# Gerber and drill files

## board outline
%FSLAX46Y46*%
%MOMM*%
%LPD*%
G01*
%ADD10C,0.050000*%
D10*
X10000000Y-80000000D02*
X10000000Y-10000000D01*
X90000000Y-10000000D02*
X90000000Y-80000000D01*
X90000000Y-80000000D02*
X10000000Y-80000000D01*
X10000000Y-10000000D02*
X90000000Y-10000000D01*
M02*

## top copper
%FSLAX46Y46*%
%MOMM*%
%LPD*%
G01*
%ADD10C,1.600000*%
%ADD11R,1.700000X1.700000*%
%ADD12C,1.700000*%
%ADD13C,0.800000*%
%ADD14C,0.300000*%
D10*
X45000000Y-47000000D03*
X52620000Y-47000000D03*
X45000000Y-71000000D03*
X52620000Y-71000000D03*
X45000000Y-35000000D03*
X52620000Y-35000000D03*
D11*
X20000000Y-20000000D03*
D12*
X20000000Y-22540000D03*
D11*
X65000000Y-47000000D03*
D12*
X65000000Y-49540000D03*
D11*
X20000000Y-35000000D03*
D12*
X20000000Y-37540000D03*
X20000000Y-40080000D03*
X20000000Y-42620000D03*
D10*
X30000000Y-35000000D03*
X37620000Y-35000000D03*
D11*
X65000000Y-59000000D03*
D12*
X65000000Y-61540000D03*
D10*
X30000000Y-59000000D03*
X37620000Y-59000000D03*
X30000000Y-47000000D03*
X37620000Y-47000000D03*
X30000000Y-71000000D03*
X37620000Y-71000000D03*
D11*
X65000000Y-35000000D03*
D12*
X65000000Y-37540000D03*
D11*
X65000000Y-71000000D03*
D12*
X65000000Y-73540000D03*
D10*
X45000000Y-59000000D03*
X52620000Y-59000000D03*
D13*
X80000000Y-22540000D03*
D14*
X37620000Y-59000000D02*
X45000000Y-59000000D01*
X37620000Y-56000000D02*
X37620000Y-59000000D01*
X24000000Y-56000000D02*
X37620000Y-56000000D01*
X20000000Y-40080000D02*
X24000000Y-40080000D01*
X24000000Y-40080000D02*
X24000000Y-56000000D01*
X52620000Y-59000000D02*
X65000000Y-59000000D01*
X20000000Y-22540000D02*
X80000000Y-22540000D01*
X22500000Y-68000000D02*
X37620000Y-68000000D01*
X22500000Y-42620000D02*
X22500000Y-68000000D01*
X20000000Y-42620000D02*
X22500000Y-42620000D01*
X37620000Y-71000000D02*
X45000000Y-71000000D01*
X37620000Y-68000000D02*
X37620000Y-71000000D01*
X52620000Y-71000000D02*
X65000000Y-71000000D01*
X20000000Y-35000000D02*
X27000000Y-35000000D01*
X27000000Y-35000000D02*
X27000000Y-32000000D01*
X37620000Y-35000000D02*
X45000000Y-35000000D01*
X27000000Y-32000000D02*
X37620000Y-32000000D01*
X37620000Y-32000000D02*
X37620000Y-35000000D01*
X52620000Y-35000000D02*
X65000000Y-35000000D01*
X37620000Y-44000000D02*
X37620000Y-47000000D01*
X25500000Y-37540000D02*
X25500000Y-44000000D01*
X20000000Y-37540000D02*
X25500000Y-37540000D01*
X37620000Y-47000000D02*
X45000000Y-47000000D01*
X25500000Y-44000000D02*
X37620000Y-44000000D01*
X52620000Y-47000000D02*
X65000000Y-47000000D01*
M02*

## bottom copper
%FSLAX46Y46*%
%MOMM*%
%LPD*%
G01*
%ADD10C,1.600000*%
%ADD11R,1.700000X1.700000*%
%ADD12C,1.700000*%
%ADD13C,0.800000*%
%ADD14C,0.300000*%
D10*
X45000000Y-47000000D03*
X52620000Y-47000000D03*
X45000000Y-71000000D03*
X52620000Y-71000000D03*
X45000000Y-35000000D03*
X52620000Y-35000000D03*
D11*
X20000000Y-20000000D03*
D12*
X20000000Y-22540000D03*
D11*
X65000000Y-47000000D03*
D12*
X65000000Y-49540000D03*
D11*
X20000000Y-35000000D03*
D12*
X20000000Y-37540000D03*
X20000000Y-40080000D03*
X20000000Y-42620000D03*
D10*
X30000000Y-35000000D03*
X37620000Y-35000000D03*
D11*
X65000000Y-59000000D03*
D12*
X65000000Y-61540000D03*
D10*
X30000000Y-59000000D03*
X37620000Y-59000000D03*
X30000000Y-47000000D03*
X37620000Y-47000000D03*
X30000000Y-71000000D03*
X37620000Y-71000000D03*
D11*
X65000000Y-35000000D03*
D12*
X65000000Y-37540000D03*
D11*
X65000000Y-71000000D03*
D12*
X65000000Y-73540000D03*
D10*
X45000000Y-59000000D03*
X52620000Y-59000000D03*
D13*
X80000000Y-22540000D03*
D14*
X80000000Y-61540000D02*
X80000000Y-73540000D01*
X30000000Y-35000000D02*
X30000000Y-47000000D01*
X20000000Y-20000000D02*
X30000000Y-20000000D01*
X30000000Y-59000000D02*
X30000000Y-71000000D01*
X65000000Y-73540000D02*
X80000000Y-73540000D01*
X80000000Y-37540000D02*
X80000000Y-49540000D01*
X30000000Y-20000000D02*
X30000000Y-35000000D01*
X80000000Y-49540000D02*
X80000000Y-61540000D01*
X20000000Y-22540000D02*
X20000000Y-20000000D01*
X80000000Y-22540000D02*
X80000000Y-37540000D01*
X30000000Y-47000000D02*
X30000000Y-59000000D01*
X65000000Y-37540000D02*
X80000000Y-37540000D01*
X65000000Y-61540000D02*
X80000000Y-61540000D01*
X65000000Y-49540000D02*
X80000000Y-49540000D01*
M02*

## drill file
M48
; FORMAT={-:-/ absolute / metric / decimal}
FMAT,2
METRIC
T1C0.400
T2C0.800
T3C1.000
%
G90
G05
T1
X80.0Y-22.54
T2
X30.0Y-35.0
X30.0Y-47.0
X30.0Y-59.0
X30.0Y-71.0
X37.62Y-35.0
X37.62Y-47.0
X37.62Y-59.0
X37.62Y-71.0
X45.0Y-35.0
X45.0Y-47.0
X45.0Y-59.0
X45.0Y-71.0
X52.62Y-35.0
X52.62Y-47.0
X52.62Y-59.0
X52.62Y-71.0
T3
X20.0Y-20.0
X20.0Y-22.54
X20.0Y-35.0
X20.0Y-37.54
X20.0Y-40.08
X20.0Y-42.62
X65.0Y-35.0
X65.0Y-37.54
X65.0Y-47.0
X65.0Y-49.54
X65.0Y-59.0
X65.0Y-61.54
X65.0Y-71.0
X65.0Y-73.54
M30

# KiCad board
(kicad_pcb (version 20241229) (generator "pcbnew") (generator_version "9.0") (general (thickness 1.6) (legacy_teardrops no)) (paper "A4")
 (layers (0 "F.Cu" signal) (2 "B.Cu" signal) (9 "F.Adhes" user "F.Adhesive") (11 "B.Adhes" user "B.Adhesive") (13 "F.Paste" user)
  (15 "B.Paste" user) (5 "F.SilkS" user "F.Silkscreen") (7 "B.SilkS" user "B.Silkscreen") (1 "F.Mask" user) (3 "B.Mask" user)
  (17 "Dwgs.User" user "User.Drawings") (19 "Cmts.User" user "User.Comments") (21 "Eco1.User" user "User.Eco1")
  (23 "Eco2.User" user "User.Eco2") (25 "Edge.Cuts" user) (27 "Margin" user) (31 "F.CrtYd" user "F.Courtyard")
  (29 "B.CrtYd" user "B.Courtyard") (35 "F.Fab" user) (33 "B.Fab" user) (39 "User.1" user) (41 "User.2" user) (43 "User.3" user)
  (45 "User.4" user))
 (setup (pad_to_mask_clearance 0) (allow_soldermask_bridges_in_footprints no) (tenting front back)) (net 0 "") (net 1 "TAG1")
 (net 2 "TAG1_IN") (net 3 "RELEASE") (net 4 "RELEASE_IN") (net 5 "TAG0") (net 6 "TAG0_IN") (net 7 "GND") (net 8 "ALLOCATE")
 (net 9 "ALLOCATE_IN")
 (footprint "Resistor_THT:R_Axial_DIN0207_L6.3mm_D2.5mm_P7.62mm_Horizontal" (layer "F.Cu") (at 45 47)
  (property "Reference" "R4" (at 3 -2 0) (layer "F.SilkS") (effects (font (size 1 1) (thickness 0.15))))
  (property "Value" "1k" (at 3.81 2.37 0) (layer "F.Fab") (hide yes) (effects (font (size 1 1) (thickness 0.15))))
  (pad "1" thru_hole circle (at 0 0) (size 1.6 1.6) (drill 0.8) (layers "*.Cu" "*.Mask") (remove_unused_layers no) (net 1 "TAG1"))
  (pad "2" thru_hole circle (at 7.62 0) (size 1.6 1.6) (drill 0.8) (layers "*.Cu" "*.Mask") (remove_unused_layers no) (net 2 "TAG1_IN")))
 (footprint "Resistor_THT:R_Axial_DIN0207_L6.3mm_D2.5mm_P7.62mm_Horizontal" (layer "F.Cu") (at 45 71)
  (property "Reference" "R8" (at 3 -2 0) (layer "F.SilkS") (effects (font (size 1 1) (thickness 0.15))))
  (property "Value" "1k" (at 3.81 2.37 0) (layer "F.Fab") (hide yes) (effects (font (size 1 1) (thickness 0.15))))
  (pad "1" thru_hole circle (at 0 0) (size 1.6 1.6) (drill 0.8) (layers "*.Cu" "*.Mask") (remove_unused_layers no) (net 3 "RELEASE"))
  (pad "2" thru_hole circle (at 7.62 0) (size 1.6 1.6) (drill 0.8) (layers "*.Cu" "*.Mask") (remove_unused_layers no) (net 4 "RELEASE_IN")))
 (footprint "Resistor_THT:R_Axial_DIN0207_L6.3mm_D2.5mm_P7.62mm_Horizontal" (layer "F.Cu") (at 45 35)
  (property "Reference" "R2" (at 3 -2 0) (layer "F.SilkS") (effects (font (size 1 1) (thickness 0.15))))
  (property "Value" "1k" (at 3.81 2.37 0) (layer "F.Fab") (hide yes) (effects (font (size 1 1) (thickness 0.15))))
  (pad "1" thru_hole circle (at 0 0) (size 1.6 1.6) (drill 0.8) (layers "*.Cu" "*.Mask") (remove_unused_layers no) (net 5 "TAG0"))
  (pad "2" thru_hole circle (at 7.62 0) (size 1.6 1.6) (drill 0.8) (layers "*.Cu" "*.Mask") (remove_unused_layers no) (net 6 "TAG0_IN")))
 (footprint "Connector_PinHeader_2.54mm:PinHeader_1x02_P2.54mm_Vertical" (layer "F.Cu") (at 20 20)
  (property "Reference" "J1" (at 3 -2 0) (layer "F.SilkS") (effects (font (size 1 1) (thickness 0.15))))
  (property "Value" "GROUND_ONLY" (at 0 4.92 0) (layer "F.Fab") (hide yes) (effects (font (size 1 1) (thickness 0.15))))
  (pad "1" thru_hole rect (at 0 0) (size 1.7 1.7) (drill 1) (layers "*.Cu" "*.Mask") (remove_unused_layers no) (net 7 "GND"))
  (pad "2" thru_hole circle (at 0 2.54) (size 1.7 1.7) (drill 1) (layers "*.Cu" "*.Mask") (remove_unused_layers no) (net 7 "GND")))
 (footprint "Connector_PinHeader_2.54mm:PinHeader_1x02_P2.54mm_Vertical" (layer "F.Cu") (at 65 47)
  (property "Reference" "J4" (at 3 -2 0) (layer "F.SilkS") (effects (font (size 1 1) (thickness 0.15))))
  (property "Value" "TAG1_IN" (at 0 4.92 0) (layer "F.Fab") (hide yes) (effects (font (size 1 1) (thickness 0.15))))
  (pad "1" thru_hole rect (at 0 0) (size 1.7 1.7) (drill 1) (layers "*.Cu" "*.Mask") (remove_unused_layers no) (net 2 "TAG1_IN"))
  (pad "2" thru_hole circle (at 0 2.54) (size 1.7 1.7) (drill 1) (layers "*.Cu" "*.Mask") (remove_unused_layers no) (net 7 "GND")))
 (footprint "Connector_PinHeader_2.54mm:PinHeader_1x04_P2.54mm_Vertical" (layer "F.Cu") (at 20 35)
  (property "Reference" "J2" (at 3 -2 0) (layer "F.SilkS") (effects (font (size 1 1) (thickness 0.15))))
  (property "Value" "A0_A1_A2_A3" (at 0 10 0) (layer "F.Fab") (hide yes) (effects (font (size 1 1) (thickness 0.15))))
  (pad "1" thru_hole rect (at 0 0) (size 1.7 1.7) (drill 1) (layers "*.Cu" "*.Mask") (remove_unused_layers no) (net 5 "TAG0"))
  (pad "2" thru_hole circle (at 0 2.54) (size 1.7 1.7) (drill 1) (layers "*.Cu" "*.Mask") (remove_unused_layers no) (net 1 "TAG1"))
  (pad "3" thru_hole circle (at 0 5.08) (size 1.7 1.7) (drill 1) (layers "*.Cu" "*.Mask") (remove_unused_layers no) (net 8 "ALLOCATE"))
  (pad "4" thru_hole circle (at 0 7.62) (size 1.7 1.7) (drill 1) (layers "*.Cu" "*.Mask") (remove_unused_layers no) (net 3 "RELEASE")))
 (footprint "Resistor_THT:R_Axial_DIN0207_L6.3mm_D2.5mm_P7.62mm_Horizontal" (layer "F.Cu") (at 30 35)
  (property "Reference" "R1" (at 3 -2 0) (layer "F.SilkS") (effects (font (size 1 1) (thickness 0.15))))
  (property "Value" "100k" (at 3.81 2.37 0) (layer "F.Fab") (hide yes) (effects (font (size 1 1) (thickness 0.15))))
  (pad "1" thru_hole circle (at 0 0) (size 1.6 1.6) (drill 0.8) (layers "*.Cu" "*.Mask") (remove_unused_layers no) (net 7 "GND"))
  (pad "2" thru_hole circle (at 7.62 0) (size 1.6 1.6) (drill 0.8) (layers "*.Cu" "*.Mask") (remove_unused_layers no) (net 5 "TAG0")))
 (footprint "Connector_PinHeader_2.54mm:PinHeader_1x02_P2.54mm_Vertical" (layer "F.Cu") (at 65 59)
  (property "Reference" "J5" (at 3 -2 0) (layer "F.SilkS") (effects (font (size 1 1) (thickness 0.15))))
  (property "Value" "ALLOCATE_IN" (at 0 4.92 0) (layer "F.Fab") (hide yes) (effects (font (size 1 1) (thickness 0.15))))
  (pad "1" thru_hole rect (at 0 0) (size 1.7 1.7) (drill 1) (layers "*.Cu" "*.Mask") (remove_unused_layers no) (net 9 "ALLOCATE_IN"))
  (pad "2" thru_hole circle (at 0 2.54) (size 1.7 1.7) (drill 1) (layers "*.Cu" "*.Mask") (remove_unused_layers no) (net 7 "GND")))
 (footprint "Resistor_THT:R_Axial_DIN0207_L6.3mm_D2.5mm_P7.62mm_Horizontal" (layer "F.Cu") (at 30 59)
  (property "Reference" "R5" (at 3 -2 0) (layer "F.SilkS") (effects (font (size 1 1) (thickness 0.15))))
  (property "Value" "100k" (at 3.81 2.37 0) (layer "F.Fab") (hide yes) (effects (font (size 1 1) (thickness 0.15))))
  (pad "1" thru_hole circle (at 0 0) (size 1.6 1.6) (drill 0.8) (layers "*.Cu" "*.Mask") (remove_unused_layers no) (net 7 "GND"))
  (pad "2" thru_hole circle (at 7.62 0) (size 1.6 1.6) (drill 0.8) (layers "*.Cu" "*.Mask") (remove_unused_layers no) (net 8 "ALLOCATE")))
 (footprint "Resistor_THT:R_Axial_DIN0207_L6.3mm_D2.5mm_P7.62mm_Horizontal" (layer "F.Cu") (at 30 47)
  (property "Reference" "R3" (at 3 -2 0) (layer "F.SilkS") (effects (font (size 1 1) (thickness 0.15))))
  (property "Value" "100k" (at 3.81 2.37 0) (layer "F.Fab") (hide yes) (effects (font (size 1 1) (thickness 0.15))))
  (pad "1" thru_hole circle (at 0 0) (size 1.6 1.6) (drill 0.8) (layers "*.Cu" "*.Mask") (remove_unused_layers no) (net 7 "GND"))
  (pad "2" thru_hole circle (at 7.62 0) (size 1.6 1.6) (drill 0.8) (layers "*.Cu" "*.Mask") (remove_unused_layers no) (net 1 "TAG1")))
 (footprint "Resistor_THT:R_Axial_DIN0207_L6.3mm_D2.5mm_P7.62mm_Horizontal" (layer "F.Cu") (at 30 71)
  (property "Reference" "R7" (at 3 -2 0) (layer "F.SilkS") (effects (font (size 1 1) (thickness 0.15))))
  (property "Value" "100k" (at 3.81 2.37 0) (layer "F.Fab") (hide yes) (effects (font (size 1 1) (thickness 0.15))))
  (pad "1" thru_hole circle (at 0 0) (size 1.6 1.6) (drill 0.8) (layers "*.Cu" "*.Mask") (remove_unused_layers no) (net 7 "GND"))
  (pad "2" thru_hole circle (at 7.62 0) (size 1.6 1.6) (drill 0.8) (layers "*.Cu" "*.Mask") (remove_unused_layers no) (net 3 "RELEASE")))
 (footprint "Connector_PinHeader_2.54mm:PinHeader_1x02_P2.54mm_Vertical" (layer "F.Cu") (at 65 35)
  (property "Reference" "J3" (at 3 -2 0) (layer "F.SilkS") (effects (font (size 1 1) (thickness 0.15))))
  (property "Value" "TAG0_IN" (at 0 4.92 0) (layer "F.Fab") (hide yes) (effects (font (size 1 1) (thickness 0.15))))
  (pad "1" thru_hole rect (at 0 0) (size 1.7 1.7) (drill 1) (layers "*.Cu" "*.Mask") (remove_unused_layers no) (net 6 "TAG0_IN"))
  (pad "2" thru_hole circle (at 0 2.54) (size 1.7 1.7) (drill 1) (layers "*.Cu" "*.Mask") (remove_unused_layers no) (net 7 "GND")))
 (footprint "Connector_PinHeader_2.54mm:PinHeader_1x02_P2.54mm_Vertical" (layer "F.Cu") (at 65 71)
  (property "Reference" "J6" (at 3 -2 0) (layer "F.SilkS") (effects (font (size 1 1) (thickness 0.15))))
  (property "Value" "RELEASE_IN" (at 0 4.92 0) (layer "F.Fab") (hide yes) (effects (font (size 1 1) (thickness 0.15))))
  (pad "1" thru_hole rect (at 0 0) (size 1.7 1.7) (drill 1) (layers "*.Cu" "*.Mask") (remove_unused_layers no) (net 4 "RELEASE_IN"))
  (pad "2" thru_hole circle (at 0 2.54) (size 1.7 1.7) (drill 1) (layers "*.Cu" "*.Mask") (remove_unused_layers no) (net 7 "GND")))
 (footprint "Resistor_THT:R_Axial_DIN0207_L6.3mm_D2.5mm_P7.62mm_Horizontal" (layer "F.Cu") (at 45 59)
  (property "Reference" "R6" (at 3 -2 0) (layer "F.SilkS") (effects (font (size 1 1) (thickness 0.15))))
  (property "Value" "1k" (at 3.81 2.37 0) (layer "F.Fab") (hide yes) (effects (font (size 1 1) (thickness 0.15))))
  (pad "1" thru_hole circle (at 0 0) (size 1.6 1.6) (drill 0.8) (layers "*.Cu" "*.Mask") (remove_unused_layers no) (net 8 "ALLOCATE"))
  (pad "2" thru_hole circle (at 7.62 0) (size 1.6 1.6) (drill 0.8) (layers "*.Cu" "*.Mask") (remove_unused_layers no) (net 9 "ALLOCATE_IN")))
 (gr_line (start 10 80) (end 10 10) (stroke (width 0.05) (type default)) (layer "Edge.Cuts"))
 (gr_line (start 90 10) (end 90 80) (stroke (width 0.05) (type default)) (layer "Edge.Cuts"))
 (gr_line (start 90 80) (end 10 80) (stroke (width 0.05) (type default)) (layer "Edge.Cuts"))
 (gr_line (start 10 10) (end 90 10) (stroke (width 0.05) (type default)) (layer "Edge.Cuts"))
 (segment (start 37.62 59) (end 45 59) (width 0.3) (layer "F.Cu") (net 8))
 (segment (start 37.62 56) (end 37.62 59) (width 0.3) (layer "F.Cu") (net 8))
 (segment (start 24 56) (end 37.62 56) (width 0.3) (layer "F.Cu") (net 8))
 (segment (start 20 40.08) (end 24 40.08) (width 0.3) (layer "F.Cu") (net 8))
 (segment (start 24 40.08) (end 24 56) (width 0.3) (layer "F.Cu") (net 8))
 (segment (start 52.62 59) (end 65 59) (width 0.3) (layer "F.Cu") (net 9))
 (segment (start 20 22.54) (end 80 22.54) (width 0.3) (layer "F.Cu") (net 7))
 (via (at 80 22.54) (size 0.8) (drill 0.4) (layers "F.Cu" "B.Cu") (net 7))
 (segment (start 80 61.54) (end 80 73.54) (width 0.3) (layer "B.Cu") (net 7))
 (segment (start 30 35) (end 30 47) (width 0.3) (layer "B.Cu") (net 7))
 (segment (start 20 20) (end 30 20) (width 0.3) (layer "B.Cu") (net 7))
 (segment (start 30 59) (end 30 71) (width 0.3) (layer "B.Cu") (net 7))
 (segment (start 65 73.54) (end 80 73.54) (width 0.3) (layer "B.Cu") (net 7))
 (segment (start 80 37.54) (end 80 49.54) (width 0.3) (layer "B.Cu") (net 7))
 (segment (start 30 20) (end 30 35) (width 0.3) (layer "B.Cu") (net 7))
 (segment (start 80 49.54) (end 80 61.54) (width 0.3) (layer "B.Cu") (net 7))
 (segment (start 20 22.54) (end 20 20) (width 0.3) (layer "B.Cu") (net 7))
 (segment (start 80 22.54) (end 80 37.54) (width 0.3) (layer "B.Cu") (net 7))
 (segment (start 30 47) (end 30 59) (width 0.3) (layer "B.Cu") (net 7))
 (segment (start 65 37.54) (end 80 37.54) (width 0.3) (layer "B.Cu") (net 7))
 (segment (start 65 61.54) (end 80 61.54) (width 0.3) (layer "B.Cu") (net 7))
 (segment (start 65 49.54) (end 80 49.54) (width 0.3) (layer "B.Cu") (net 7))
 (segment (start 22.5 68) (end 37.62 68) (width 0.3) (layer "F.Cu") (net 3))
 (segment (start 22.5 42.62) (end 22.5 68) (width 0.3) (layer "F.Cu") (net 3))
 (segment (start 20 42.62) (end 22.5 42.62) (width 0.3) (layer "F.Cu") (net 3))
 (segment (start 37.62 71) (end 45 71) (width 0.3) (layer "F.Cu") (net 3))
 (segment (start 37.62 68) (end 37.62 71) (width 0.3) (layer "F.Cu") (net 3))
 (segment (start 52.62 71) (end 65 71) (width 0.3) (layer "F.Cu") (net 4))
 (segment (start 20 35) (end 27 35) (width 0.3) (layer "F.Cu") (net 5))
 (segment (start 27 35) (end 27 32) (width 0.3) (layer "F.Cu") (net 5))
 (segment (start 37.62 35) (end 45 35) (width 0.3) (layer "F.Cu") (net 5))
 (segment (start 27 32) (end 37.62 32) (width 0.3) (layer "F.Cu") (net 5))
 (segment (start 37.62 32) (end 37.62 35) (width 0.3) (layer "F.Cu") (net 5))
 (segment (start 52.62 35) (end 65 35) (width 0.3) (layer "F.Cu") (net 6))
 (segment (start 37.62 44) (end 37.62 47) (width 0.3) (layer "F.Cu") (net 1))
 (segment (start 25.5 37.54) (end 25.5 44) (width 0.3) (layer "F.Cu") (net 1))
 (segment (start 20 37.54) (end 25.5 37.54) (width 0.3) (layer "F.Cu") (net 1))
 (segment (start 37.62 47) (end 45 47) (width 0.3) (layer "F.Cu") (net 1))
 (segment (start 25.5 44) (end 37.62 44) (width 0.3) (layer "F.Cu") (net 1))
 (segment (start 52.62 47) (end 65 47) (width 0.3) (layer "F.Cu") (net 2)))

